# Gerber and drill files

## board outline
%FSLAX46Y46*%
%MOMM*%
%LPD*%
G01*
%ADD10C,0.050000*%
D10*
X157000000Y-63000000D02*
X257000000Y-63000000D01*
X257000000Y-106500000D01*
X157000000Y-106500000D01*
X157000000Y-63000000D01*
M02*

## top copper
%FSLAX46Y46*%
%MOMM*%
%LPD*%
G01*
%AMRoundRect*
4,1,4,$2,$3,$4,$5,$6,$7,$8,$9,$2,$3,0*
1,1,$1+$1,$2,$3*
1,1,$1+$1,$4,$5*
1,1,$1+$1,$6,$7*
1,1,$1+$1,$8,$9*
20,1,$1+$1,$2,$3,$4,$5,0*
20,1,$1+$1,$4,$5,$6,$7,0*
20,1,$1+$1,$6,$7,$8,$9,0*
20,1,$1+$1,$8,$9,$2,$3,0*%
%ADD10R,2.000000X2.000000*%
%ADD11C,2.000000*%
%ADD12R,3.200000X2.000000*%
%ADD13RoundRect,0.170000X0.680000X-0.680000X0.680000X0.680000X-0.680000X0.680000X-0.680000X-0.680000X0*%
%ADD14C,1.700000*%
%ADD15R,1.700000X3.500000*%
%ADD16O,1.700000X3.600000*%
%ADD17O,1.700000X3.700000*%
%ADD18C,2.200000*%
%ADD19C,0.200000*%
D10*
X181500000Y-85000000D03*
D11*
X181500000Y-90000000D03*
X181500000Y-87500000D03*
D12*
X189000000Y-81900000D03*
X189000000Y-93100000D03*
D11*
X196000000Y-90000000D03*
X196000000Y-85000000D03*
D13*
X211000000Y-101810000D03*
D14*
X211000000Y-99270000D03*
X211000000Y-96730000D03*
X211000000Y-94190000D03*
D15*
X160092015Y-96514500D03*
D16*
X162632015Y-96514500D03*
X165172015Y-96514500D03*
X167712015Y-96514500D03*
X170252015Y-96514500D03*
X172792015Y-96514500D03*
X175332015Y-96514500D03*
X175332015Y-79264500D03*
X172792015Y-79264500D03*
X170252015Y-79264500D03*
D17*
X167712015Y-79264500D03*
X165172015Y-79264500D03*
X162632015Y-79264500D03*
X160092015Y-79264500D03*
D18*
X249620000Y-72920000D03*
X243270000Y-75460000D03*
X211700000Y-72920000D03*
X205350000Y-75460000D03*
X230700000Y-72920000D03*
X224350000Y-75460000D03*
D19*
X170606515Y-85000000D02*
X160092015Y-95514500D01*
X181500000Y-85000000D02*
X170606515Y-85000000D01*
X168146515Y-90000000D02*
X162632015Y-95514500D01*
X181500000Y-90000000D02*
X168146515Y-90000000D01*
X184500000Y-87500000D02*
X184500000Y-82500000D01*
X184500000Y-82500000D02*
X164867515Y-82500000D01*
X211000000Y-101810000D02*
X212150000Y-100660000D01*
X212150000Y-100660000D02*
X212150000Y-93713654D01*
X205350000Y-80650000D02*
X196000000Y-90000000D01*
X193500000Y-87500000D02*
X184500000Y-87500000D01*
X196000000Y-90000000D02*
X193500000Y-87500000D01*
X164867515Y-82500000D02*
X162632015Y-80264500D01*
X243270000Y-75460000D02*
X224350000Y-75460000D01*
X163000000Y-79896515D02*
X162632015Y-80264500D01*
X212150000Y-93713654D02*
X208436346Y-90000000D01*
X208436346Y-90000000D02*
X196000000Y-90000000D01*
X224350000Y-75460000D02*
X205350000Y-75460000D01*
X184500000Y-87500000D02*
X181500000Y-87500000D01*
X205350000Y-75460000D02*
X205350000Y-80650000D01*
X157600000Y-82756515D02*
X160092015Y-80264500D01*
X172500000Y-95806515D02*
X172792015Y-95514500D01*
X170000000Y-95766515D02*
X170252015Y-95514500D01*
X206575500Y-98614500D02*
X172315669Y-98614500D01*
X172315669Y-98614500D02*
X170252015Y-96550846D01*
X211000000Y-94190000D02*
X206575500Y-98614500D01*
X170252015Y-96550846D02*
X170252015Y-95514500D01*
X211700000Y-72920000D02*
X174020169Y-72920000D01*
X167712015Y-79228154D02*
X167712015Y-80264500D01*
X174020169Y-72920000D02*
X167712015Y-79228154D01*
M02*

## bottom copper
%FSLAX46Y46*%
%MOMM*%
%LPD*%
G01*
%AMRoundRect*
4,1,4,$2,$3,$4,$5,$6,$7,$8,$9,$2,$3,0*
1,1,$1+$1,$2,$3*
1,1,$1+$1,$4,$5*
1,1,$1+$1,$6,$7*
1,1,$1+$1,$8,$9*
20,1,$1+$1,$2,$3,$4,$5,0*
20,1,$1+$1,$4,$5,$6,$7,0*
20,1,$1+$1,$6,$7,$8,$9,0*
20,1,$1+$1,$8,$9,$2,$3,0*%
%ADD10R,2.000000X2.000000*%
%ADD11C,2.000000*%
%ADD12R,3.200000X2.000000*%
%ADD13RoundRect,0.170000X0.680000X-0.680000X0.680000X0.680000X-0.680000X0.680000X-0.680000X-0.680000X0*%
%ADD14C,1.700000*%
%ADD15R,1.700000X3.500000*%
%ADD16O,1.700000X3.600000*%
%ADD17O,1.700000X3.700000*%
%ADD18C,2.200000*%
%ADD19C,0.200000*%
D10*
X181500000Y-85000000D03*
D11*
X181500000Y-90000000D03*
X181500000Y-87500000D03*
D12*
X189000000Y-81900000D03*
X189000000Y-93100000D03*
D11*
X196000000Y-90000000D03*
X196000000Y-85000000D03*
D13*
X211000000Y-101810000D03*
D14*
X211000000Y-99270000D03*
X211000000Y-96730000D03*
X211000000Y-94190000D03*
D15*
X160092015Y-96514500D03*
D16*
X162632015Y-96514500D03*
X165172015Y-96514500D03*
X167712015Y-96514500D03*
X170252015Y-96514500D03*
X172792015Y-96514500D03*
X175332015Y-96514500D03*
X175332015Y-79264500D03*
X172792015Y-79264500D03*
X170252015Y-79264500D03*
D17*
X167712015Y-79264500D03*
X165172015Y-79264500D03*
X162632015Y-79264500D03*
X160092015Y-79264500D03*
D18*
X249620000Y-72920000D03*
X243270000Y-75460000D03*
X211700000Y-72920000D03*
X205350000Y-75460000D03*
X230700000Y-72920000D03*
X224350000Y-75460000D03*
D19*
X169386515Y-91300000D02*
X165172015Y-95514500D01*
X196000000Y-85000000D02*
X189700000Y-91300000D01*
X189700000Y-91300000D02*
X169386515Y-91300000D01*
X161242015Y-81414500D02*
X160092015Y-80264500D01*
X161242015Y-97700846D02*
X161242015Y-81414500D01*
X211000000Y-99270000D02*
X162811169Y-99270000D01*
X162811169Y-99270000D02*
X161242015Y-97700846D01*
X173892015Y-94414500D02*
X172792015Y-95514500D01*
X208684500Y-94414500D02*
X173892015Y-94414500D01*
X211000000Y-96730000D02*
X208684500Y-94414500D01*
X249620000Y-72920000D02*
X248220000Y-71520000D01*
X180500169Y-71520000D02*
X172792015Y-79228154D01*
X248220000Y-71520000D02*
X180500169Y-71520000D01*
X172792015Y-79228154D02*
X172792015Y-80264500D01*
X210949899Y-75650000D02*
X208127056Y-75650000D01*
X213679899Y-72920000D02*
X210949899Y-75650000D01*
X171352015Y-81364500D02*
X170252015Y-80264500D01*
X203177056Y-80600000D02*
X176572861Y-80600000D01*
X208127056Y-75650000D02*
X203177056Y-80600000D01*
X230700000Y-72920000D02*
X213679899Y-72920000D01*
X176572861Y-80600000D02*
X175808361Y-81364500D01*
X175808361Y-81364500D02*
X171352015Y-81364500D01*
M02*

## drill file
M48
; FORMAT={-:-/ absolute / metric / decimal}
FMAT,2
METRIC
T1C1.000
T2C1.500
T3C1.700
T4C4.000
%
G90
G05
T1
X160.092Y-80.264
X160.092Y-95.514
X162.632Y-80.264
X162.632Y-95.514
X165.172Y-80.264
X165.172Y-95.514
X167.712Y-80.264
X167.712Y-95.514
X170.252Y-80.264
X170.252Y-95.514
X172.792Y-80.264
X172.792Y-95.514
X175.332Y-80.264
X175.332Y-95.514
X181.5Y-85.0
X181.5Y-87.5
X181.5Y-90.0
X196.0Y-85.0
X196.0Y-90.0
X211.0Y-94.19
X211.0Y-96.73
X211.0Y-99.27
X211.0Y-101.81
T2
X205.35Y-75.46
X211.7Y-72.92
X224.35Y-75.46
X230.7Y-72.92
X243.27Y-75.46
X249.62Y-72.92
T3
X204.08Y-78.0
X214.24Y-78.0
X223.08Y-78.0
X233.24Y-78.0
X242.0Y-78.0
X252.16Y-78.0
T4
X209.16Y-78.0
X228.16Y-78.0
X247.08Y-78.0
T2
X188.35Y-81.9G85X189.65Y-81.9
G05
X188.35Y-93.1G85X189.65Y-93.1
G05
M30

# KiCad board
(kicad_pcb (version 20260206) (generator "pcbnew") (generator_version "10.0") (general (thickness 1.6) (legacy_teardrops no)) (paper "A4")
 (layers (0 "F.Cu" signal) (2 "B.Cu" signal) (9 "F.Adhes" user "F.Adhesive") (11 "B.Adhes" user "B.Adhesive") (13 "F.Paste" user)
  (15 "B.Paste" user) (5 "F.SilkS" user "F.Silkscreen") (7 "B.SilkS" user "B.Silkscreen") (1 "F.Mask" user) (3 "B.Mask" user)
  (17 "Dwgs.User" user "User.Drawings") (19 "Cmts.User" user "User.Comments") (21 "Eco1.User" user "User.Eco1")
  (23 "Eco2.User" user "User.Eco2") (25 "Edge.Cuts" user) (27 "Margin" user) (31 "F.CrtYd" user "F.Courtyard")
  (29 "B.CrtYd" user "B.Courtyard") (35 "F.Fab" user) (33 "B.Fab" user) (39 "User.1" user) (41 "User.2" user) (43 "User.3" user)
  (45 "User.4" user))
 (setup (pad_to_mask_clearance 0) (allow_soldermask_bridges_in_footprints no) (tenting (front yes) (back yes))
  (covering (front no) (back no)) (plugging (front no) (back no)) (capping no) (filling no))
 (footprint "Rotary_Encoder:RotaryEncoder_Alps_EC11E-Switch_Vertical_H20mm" (layer "F.Cu") (at 181.5 85)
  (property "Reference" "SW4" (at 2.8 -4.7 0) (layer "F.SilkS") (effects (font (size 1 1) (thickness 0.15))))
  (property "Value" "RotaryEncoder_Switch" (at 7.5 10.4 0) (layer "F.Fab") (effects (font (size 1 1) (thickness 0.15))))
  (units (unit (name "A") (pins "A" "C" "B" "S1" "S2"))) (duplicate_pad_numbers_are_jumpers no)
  (pad "A" thru_hole rect (at 0 0) (size 2 2) (drill 1) (layers "*.Cu" "*.Mask") (remove_unused_layers no) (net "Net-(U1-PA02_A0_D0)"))
  (pad "B" thru_hole circle (at 0 5) (size 2 2) (drill 1) (layers "*.Cu" "*.Mask") (remove_unused_layers no) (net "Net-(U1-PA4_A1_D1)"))
  (pad "C" thru_hole circle (at 0 2.5) (size 2 2) (drill 1) (layers "*.Cu" "*.Mask") (remove_unused_layers no) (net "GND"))
  (pad "MP" thru_hole rect (at 7.5 -3.1) (size 3.2 2) (drill oval 2.8 1.5) (layers "*.Cu" "*.Mask") (remove_unused_layers no))
  (pad "MP" thru_hole rect (at 7.5 8.1) (size 3.2 2) (drill oval 2.8 1.5) (layers "*.Cu" "*.Mask") (remove_unused_layers no))
  (pad "S1" thru_hole circle (at 14.5 5) (size 2 2) (drill 1) (layers "*.Cu" "*.Mask") (remove_unused_layers no) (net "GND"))
  (pad "S2" thru_hole circle (at 14.5 0) (size 2 2) (drill 1) (layers "*.Cu" "*.Mask") (remove_unused_layers no) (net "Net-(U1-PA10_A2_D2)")))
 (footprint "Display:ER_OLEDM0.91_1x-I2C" (layer "F.Cu") (at 211 101.81 90)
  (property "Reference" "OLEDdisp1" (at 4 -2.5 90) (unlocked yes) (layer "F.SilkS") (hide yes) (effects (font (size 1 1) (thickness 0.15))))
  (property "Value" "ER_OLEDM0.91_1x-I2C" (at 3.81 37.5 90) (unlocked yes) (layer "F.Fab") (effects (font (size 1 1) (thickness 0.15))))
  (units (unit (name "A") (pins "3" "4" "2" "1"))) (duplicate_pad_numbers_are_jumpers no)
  (pad "1" thru_hole roundrect (at 0 0 90) (size 1.7 1.7) (drill 1) (layers "*.Cu" "*.Mask") (remove_unused_layers no)
   (roundrect_rratio 0.1) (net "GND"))
  (pad "2" thru_hole circle (at 2.54 0 90) (size 1.7 1.7) (drill 1) (layers "*.Cu" "*.Mask") (remove_unused_layers no)
   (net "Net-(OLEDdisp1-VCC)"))
  (pad "3" thru_hole circle (at 5.08 0 90) (size 1.7 1.7) (drill 1) (layers "*.Cu" "*.Mask") (remove_unused_layers no)
   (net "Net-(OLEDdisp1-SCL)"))
  (pad "4" thru_hole circle (at 7.62 0 90) (size 1.7 1.7) (drill 1) (layers "*.Cu" "*.Mask") (remove_unused_layers no)
   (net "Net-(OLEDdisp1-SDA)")))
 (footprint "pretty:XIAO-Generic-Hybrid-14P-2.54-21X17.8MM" (layer "F.Cu") (at 167.712015 87.8895 90)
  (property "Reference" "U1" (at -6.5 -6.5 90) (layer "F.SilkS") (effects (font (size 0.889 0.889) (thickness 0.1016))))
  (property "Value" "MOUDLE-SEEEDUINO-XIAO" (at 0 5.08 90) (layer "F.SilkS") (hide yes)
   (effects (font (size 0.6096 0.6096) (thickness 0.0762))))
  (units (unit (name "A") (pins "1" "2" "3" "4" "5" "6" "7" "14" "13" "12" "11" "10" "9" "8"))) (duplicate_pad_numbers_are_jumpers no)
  (pad "1" thru_hole rect (at -7.625 -7.62 90) (size 3.5 1.7) (drill 1 (offset -1 0)) (layers "*.Cu" "*.Mask") (remove_unused_layers no)
   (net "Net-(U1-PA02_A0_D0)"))
  (pad "2" thru_hole oval (at -7.625 -5.08 90) (size 3.6 1.7) (drill 1 (offset -1 0)) (layers "*.Cu" "*.Mask") (remove_unused_layers no)
   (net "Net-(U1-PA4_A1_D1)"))
  (pad "3" thru_hole oval (at -7.625 -2.54 90) (size 3.6 1.7) (drill 1 (offset -1 0)) (layers "*.Cu" "*.Mask") (remove_unused_layers no)
   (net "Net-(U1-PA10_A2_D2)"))
  (pad "4" thru_hole oval (at -7.625 0 90) (size 3.6 1.7) (drill 1 (offset -1 0)) (layers "*.Cu" "*.Mask") (remove_unused_layers no)
   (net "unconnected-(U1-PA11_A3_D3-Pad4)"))
  (pad "5" thru_hole oval (at -7.625 2.54 90) (size 3.6 1.7) (drill 1 (offset -1 0)) (layers "*.Cu" "*.Mask") (remove_unused_layers no)
   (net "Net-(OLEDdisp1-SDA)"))
  (pad "6" thru_hole oval (at -7.625 5.08 270) (size 3.6 1.7) (drill 1 (offset 1 0)) (layers "*.Cu" "*.Mask") (remove_unused_layers no)
   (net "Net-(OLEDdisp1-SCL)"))
  (pad "7" thru_hole oval (at -7.625 7.62 90) (size 3.6 1.7) (drill 1 (offset -1 0)) (layers "*.Cu" "*.Mask") (remove_unused_layers no)
   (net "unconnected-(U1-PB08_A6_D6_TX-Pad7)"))
  (pad "8" thru_hole oval (at 7.625 7.62 90) (size 3.6 1.7) (drill 1 (offset 1 0)) (layers "*.Cu" "*.Mask") (remove_unused_layers no)
   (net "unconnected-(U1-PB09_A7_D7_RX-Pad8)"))
  (pad "9" thru_hole oval (at 7.625 5.08 90) (size 3.6 1.7) (drill 1 (offset 1 0)) (layers "*.Cu" "*.Mask") (remove_unused_layers no)
   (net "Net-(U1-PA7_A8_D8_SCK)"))
  (pad "10" thru_hole oval (at 7.625 2.54 90) (size 3.6 1.7) (drill 1 (offset 1 0)) (layers "*.Cu" "*.Mask") (remove_unused_layers no)
   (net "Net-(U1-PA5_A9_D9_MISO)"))
  (pad "11" thru_hole oval (at 7.625 0 90) (size 3.7 1.7) (drill 1 (offset 1 0)) (layers "*.Cu" "*.Mask") (remove_unused_layers no)
   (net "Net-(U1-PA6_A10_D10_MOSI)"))
  (pad "12" thru_hole oval (at 7.625 -2.54 90) (size 3.7 1.7) (drill 1 (offset 1 0)) (layers "*.Cu" "*.Mask") (remove_unused_layers no)
   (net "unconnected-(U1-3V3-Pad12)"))
  (pad "13" thru_hole oval (at 7.625 -5.08 90) (size 3.7 1.7) (drill 1 (offset 1 0)) (layers "*.Cu" "*.Mask") (remove_unused_layers no)
   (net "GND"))
  (pad "14" thru_hole oval (at 7.625 -7.62 90) (size 3.7 1.7) (drill 1 (offset 1 0)) (layers "*.Cu" "*.Mask") (remove_unused_layers no)
   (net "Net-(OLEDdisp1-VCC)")))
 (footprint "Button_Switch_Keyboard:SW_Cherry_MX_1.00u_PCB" (layer "F.Cu") (at 249.62 72.92)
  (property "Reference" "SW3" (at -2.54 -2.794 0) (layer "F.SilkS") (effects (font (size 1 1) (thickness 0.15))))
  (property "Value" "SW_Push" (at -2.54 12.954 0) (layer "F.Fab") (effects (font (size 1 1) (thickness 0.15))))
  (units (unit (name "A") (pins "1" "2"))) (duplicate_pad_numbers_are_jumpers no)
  (pad "" np_thru_hole circle (at -7.62 5.08) (size 1.7 1.7) (drill 1.7) (layers "*.Cu" "*.Mask"))
  (pad "" np_thru_hole circle (at -2.54 5.08) (size 4 4) (drill 4) (layers "*.Cu" "*.Mask"))
  (pad "" np_thru_hole circle (at 2.54 5.08) (size 1.7 1.7) (drill 1.7) (layers "*.Cu" "*.Mask"))
  (pad "1" thru_hole circle (at 0 0) (size 2.2 2.2) (drill 1.5) (layers "*.Cu" "*.Mask") (remove_unused_layers no)
   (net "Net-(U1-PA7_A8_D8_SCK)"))
  (pad "2" thru_hole circle (at -6.35 2.54) (size 2.2 2.2) (drill 1.5) (layers "*.Cu" "*.Mask") (remove_unused_layers no) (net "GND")))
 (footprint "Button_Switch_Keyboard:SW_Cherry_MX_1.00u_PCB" (layer "F.Cu") (at 211.7 72.92)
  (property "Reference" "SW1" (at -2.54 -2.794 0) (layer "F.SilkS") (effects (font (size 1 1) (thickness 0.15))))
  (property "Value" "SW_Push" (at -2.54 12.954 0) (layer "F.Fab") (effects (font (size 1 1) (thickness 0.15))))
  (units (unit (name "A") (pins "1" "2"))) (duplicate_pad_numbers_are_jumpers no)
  (pad "" np_thru_hole circle (at -7.62 5.08) (size 1.7 1.7) (drill 1.7) (layers "*.Cu" "*.Mask"))
  (pad "" np_thru_hole circle (at -2.54 5.08) (size 4 4) (drill 4) (layers "*.Cu" "*.Mask"))
  (pad "" np_thru_hole circle (at 2.54 5.08) (size 1.7 1.7) (drill 1.7) (layers "*.Cu" "*.Mask"))
  (pad "1" thru_hole circle (at 0 0) (size 2.2 2.2) (drill 1.5) (layers "*.Cu" "*.Mask") (remove_unused_layers no)
   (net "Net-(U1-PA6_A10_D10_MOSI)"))
  (pad "2" thru_hole circle (at -6.35 2.54) (size 2.2 2.2) (drill 1.5) (layers "*.Cu" "*.Mask") (remove_unused_layers no) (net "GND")))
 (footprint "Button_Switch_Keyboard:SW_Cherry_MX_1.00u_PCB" (layer "F.Cu") (at 230.7 72.92)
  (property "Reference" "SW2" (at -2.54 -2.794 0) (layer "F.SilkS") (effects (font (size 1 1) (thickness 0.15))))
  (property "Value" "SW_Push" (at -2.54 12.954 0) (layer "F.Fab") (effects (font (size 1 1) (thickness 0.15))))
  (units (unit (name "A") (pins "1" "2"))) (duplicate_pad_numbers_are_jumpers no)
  (pad "" np_thru_hole circle (at -7.62 5.08) (size 1.7 1.7) (drill 1.7) (layers "*.Cu" "*.Mask"))
  (pad "" np_thru_hole circle (at -2.54 5.08) (size 4 4) (drill 4) (layers "*.Cu" "*.Mask"))
  (pad "" np_thru_hole circle (at 2.54 5.08) (size 1.7 1.7) (drill 1.7) (layers "*.Cu" "*.Mask"))
  (pad "1" thru_hole circle (at 0 0) (size 2.2 2.2) (drill 1.5) (layers "*.Cu" "*.Mask") (remove_unused_layers no)
   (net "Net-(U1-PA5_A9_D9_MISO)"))
  (pad "2" thru_hole circle (at -6.35 2.54) (size 2.2 2.2) (drill 1.5) (layers "*.Cu" "*.Mask") (remove_unused_layers no) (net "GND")))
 (gr_rect (start 157 63) (end 257 106.5) (stroke (width 0.05) (type default)) (fill no) (layer "Edge.Cuts"))
 (segment (start 170.606515 85) (end 160.092015 95.5145) (width 0.2) (layer "F.Cu") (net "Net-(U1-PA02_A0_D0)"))
 (segment (start 181.5 85) (end 170.606515 85) (width 0.2) (layer "F.Cu") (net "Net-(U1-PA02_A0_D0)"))
 (segment (start 168.146515 90) (end 162.632015 95.5145) (width 0.2) (layer "F.Cu") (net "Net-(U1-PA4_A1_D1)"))
 (segment (start 181.5 90) (end 168.146515 90) (width 0.2) (layer "F.Cu") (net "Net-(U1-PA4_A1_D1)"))
 (segment (start 184.5 87.5) (end 184.5 82.5) (width 0.2) (layer "F.Cu") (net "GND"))
 (segment (start 184.5 82.5) (end 164.867515 82.5) (width 0.2) (layer "F.Cu") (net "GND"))
 (segment (start 211 101.81) (end 212.15 100.66) (width 0.2) (layer "F.Cu") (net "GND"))
 (segment (start 212.15 100.66) (end 212.15 93.713654) (width 0.2) (layer "F.Cu") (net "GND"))
 (segment (start 205.35 80.65) (end 196 90) (width 0.2) (layer "F.Cu") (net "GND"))
 (segment (start 193.5 87.5) (end 184.5 87.5) (width 0.2) (layer "F.Cu") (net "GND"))
 (segment (start 196 90) (end 193.5 87.5) (width 0.2) (layer "F.Cu") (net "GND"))
 (segment (start 164.867515 82.5) (end 162.632015 80.2645) (width 0.2) (layer "F.Cu") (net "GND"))
 (segment (start 243.27 75.46) (end 224.35 75.46) (width 0.2) (layer "F.Cu") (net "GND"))
 (segment (start 163 79.896515) (end 162.632015 80.2645) (width 0.2) (layer "F.Cu") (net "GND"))
 (segment (start 212.15 93.713654) (end 208.436346 90) (width 0.2) (layer "F.Cu") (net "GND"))
 (segment (start 208.436346 90) (end 196 90) (width 0.2) (layer "F.Cu") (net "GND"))
 (segment (start 224.35 75.46) (end 205.35 75.46) (width 0.2) (layer "F.Cu") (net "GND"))
 (segment (start 184.5 87.5) (end 181.5 87.5) (width 0.2) (layer "F.Cu") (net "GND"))
 (segment (start 205.35 75.46) (end 205.35 80.65) (width 0.2) (layer "F.Cu") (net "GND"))
 (segment (start 169.386515 91.3) (end 165.172015 95.5145) (width 0.2) (layer "B.Cu") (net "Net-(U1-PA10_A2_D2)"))
 (segment (start 196 85) (end 189.7 91.3) (width 0.2) (layer "B.Cu") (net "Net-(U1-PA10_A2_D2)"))
 (segment (start 189.7 91.3) (end 169.386515 91.3) (width 0.2) (layer "B.Cu") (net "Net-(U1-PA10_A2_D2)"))
 (segment (start 157.6 82.756515) (end 160.092015 80.2645) (width 0.2) (layer "F.Cu") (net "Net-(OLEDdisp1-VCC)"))
 (segment (start 161.242015 81.4145) (end 160.092015 80.2645) (width 0.2) (layer "B.Cu") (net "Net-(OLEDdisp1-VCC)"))
 (segment (start 161.242015 97.700846) (end 161.242015 81.4145) (width 0.2) (layer "B.Cu") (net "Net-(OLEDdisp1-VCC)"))
 (segment (start 211 99.27) (end 162.811169 99.27) (width 0.2) (layer "B.Cu") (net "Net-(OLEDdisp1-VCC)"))
 (segment (start 162.811169 99.27) (end 161.242015 97.700846) (width 0.2) (layer "B.Cu") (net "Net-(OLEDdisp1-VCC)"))
 (segment (start 172.5 95.806515) (end 172.792015 95.5145) (width 0.2) (layer "F.Cu") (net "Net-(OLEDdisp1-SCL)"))
 (segment (start 173.892015 94.4145) (end 172.792015 95.5145) (width 0.2) (layer "B.Cu") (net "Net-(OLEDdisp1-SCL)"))
 (segment (start 208.6845 94.4145) (end 173.892015 94.4145) (width 0.2) (layer "B.Cu") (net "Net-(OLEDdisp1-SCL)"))
 (segment (start 211 96.73) (end 208.6845 94.4145) (width 0.2) (layer "B.Cu") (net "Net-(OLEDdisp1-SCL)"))
 (segment (start 170 95.766515) (end 170.252015 95.5145) (width 0.2) (layer "F.Cu") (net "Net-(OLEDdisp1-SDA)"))
 (segment (start 206.5755 98.6145) (end 172.315669 98.6145) (width 0.2) (layer "F.Cu") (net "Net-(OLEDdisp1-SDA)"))
 (segment (start 172.315669 98.6145) (end 170.252015 96.550846) (width 0.2) (layer "F.Cu") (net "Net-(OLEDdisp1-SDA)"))
 (segment (start 211 94.19) (end 206.5755 98.6145) (width 0.2) (layer "F.Cu") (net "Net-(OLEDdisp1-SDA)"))
 (segment (start 170.252015 96.550846) (end 170.252015 95.5145) (width 0.2) (layer "F.Cu") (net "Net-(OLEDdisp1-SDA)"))
 (segment (start 249.62 72.92) (end 248.22 71.52) (width 0.2) (layer "B.Cu") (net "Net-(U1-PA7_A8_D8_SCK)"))
 (segment (start 180.500169 71.52) (end 172.792015 79.228154) (width 0.2) (layer "B.Cu") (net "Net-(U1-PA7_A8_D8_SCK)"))
 (segment (start 248.22 71.52) (end 180.500169 71.52) (width 0.2) (layer "B.Cu") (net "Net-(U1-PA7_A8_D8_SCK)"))
 (segment (start 172.792015 79.228154) (end 172.792015 80.2645) (width 0.2) (layer "B.Cu") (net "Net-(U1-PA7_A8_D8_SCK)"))
 (segment (start 210.949899 75.65) (end 208.127056 75.65) (width 0.2) (layer "B.Cu") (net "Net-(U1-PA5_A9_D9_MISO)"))
 (segment (start 213.679899 72.92) (end 210.949899 75.65) (width 0.2) (layer "B.Cu") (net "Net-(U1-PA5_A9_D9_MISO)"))
 (segment (start 171.352015 81.3645) (end 170.252015 80.2645) (width 0.2) (layer "B.Cu") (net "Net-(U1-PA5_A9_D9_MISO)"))
 (segment (start 203.177056 80.6) (end 176.572861 80.6) (width 0.2) (layer "B.Cu") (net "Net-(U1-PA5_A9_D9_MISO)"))
 (segment (start 208.127056 75.65) (end 203.177056 80.6) (width 0.2) (layer "B.Cu") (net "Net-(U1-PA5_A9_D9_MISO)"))
 (segment (start 230.7 72.92) (end 213.679899 72.92) (width 0.2) (layer "B.Cu") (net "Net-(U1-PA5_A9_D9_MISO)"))
 (segment (start 176.572861 80.6) (end 175.808361 81.3645) (width 0.2) (layer "B.Cu") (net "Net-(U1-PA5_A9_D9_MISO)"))
 (segment (start 175.808361 81.3645) (end 171.352015 81.3645) (width 0.2) (layer "B.Cu") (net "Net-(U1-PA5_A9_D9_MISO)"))
 (segment (start 211.7 72.92) (end 174.020169 72.92) (width 0.2) (layer "F.Cu") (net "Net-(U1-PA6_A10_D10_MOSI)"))
 (segment (start 167.712015 79.228154) (end 167.712015 80.2645) (width 0.2) (layer "F.Cu") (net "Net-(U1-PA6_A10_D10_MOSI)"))
 (segment (start 174.020169 72.92) (end 167.712015 79.228154) (width 0.2) (layer "F.Cu") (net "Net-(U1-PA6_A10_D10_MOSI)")))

